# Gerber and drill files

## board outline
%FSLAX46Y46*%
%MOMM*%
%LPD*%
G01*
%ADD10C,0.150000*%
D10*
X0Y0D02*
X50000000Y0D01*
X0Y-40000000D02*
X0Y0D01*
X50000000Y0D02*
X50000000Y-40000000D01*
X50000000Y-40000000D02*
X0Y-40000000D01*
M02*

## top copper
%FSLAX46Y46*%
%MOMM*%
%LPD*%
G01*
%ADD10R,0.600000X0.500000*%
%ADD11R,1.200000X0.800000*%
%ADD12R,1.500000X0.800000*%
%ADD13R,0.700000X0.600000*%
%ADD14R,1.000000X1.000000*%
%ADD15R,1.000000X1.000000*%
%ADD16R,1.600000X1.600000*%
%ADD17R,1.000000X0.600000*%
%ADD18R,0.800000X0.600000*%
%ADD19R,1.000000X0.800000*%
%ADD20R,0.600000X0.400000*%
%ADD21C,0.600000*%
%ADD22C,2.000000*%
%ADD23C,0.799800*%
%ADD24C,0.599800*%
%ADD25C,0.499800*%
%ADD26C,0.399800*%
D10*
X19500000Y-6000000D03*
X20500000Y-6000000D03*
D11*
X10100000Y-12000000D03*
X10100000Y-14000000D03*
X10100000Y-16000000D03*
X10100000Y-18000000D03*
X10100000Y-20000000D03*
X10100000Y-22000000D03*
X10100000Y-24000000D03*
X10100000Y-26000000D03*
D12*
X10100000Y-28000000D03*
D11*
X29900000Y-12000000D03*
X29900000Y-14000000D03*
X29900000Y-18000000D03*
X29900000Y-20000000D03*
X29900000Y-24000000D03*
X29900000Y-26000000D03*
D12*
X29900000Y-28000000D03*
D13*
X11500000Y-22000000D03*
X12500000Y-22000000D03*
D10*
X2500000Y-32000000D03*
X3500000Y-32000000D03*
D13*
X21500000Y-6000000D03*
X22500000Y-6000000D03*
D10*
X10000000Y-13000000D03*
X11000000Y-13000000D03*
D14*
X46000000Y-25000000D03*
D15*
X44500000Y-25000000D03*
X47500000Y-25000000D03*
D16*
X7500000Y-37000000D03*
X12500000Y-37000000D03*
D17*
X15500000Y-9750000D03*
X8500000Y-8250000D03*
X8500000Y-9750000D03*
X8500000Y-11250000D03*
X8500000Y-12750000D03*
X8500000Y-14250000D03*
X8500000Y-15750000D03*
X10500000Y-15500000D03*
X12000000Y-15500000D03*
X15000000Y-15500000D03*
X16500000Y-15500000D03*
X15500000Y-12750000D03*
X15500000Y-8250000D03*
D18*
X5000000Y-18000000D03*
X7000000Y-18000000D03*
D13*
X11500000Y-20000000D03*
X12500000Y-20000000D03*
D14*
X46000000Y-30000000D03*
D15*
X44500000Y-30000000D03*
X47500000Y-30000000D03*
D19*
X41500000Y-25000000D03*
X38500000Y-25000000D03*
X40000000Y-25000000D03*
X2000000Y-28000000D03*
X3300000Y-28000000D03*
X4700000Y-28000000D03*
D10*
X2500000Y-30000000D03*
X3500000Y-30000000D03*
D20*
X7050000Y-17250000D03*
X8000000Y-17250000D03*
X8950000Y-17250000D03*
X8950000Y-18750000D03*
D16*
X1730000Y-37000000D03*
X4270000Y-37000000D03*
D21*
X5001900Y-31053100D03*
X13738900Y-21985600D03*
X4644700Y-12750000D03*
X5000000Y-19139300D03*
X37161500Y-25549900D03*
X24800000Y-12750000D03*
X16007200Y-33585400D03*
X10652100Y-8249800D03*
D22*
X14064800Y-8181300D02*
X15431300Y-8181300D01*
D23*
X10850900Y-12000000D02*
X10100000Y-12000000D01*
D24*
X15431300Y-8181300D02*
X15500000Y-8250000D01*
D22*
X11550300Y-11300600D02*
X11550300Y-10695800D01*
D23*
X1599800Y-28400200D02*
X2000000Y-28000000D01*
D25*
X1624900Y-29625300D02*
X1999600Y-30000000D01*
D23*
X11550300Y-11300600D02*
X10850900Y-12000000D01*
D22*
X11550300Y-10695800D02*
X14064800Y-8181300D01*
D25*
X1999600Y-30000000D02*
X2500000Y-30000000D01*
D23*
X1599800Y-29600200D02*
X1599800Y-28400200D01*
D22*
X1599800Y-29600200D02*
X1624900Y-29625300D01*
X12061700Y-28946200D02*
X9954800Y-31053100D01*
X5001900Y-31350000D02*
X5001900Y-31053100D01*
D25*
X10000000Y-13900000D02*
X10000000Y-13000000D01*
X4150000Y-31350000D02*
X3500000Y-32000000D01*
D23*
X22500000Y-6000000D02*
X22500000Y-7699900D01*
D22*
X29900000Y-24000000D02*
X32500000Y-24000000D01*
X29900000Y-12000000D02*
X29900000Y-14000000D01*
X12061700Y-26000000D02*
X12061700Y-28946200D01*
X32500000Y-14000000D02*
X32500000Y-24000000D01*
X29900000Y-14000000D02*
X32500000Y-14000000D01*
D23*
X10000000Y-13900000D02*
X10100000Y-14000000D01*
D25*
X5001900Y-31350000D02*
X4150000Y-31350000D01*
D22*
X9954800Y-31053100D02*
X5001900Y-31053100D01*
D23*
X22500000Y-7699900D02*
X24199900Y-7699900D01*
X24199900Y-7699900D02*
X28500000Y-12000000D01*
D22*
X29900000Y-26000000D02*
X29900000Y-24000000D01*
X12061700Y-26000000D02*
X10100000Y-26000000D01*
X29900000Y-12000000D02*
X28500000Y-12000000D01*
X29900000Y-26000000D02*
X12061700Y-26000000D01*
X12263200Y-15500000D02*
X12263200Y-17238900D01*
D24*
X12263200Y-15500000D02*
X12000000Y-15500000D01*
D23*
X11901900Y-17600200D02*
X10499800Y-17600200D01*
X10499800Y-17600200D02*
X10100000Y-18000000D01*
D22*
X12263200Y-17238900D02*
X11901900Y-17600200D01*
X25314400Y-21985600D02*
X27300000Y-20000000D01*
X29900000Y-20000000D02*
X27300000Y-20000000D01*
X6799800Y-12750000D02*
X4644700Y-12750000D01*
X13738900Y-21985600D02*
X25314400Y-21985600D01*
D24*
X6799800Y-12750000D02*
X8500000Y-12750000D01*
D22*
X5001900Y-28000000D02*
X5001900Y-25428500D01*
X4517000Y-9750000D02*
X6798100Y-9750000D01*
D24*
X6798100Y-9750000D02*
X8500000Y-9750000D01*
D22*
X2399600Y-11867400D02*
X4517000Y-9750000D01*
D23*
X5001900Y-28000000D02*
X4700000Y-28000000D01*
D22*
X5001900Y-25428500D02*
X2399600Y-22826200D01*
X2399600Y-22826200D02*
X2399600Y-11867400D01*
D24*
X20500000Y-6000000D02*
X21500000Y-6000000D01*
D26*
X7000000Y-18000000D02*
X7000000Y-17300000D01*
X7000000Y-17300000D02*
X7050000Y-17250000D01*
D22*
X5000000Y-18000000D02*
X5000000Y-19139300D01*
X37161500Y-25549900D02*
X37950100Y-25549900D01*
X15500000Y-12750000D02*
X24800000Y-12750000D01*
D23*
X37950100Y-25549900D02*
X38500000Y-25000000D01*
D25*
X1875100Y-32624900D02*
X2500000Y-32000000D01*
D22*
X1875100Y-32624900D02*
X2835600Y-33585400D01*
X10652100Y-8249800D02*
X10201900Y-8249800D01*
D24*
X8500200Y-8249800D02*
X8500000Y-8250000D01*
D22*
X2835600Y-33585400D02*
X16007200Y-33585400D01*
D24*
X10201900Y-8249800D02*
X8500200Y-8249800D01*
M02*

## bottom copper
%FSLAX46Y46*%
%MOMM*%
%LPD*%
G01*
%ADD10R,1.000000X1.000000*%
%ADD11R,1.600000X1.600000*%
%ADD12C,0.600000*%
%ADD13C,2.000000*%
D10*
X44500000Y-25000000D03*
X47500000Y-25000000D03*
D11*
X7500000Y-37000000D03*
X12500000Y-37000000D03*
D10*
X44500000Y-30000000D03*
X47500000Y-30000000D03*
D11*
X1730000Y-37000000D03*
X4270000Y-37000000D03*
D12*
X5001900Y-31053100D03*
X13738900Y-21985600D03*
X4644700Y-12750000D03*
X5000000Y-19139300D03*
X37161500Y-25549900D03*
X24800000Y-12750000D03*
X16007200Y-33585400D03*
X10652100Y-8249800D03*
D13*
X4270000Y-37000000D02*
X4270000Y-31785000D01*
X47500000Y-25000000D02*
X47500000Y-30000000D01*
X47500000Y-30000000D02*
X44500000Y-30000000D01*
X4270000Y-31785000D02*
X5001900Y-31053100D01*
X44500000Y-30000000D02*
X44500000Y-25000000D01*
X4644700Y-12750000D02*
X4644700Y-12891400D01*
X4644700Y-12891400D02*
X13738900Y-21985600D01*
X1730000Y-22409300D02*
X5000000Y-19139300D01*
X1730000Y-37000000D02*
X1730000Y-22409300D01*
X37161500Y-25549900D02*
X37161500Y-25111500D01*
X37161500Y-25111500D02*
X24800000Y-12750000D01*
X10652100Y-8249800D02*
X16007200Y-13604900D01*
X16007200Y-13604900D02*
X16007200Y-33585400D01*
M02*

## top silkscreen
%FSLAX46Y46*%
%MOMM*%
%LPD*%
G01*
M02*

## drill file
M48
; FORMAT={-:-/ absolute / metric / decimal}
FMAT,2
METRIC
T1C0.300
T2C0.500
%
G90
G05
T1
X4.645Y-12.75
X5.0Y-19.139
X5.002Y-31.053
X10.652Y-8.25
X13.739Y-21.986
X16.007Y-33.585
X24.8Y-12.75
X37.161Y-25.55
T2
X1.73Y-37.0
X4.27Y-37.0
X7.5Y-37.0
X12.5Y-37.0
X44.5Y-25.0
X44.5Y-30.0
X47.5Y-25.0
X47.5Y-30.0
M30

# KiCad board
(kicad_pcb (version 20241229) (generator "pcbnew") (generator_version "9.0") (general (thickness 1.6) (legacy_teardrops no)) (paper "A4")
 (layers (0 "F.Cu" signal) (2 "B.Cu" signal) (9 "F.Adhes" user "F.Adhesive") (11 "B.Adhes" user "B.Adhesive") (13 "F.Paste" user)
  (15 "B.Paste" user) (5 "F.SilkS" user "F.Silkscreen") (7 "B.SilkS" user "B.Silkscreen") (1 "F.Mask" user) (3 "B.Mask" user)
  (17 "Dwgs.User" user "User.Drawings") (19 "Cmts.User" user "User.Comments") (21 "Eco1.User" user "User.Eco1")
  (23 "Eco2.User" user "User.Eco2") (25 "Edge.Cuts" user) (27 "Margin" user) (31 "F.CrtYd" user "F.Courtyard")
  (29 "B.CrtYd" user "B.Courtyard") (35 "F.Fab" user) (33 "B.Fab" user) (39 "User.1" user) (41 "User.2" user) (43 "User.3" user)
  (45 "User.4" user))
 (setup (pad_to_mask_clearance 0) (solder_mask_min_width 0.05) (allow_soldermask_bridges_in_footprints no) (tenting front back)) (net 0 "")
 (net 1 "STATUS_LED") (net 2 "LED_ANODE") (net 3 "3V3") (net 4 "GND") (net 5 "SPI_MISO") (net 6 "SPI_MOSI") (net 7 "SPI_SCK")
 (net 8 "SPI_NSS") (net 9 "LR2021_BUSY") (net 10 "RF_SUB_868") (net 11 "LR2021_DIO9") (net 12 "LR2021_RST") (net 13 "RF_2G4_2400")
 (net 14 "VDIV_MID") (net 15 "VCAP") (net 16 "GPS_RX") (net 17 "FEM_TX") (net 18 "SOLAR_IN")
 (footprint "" (layer "F.Cu") (at 20 6)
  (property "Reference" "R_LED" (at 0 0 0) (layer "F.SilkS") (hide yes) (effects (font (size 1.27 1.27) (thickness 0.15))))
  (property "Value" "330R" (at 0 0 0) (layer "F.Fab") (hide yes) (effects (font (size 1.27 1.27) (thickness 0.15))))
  (pad "1" smd rect (at -0.5 0) (size 0.6 0.5) (layers "F.Cu" "F.Mask") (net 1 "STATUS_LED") (thermal_bridge_angle 45))
  (pad "2" smd rect (at 0.5 0) (size 0.6 0.5) (layers "F.Cu" "F.Mask") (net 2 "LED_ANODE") (thermal_bridge_angle 45)))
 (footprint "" (layer "F.Cu") (at 20 20)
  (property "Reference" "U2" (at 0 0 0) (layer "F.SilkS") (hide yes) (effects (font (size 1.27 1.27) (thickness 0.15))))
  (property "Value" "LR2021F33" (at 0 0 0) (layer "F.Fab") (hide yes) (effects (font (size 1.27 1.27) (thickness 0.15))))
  (pad "1" smd rect (at -9.9 -8) (size 1.2 0.8) (layers "F.Cu" "F.Mask") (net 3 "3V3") (thermal_bridge_angle 45))
  (pad "2" smd rect (at -9.9 -6) (size 1.2 0.8) (layers "F.Cu" "F.Mask") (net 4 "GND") (thermal_bridge_angle 45))
  (pad "3" smd rect (at -9.9 -4) (size 1.2 0.8) (layers "F.Cu" "F.Mask") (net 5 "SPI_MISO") (thermal_bridge_angle 45))
  (pad "4" smd rect (at -9.9 -2) (size 1.2 0.8) (layers "F.Cu" "F.Mask") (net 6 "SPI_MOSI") (thermal_bridge_angle 45))
  (pad "5" smd rect (at -9.9 0) (size 1.2 0.8) (layers "F.Cu" "F.Mask") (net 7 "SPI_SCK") (thermal_bridge_angle 45))
  (pad "6" smd rect (at -9.9 2) (size 1.2 0.8) (layers "F.Cu" "F.Mask") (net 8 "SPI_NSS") (thermal_bridge_angle 45))
  (pad "7" smd rect (at -9.9 4) (size 1.2 0.8) (layers "F.Cu" "F.Mask") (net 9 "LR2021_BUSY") (thermal_bridge_angle 45))
  (pad "8" smd rect (at -9.9 6) (size 1.2 0.8) (layers "F.Cu" "F.Mask") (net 4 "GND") (thermal_bridge_angle 45))
  (pad "9" smd rect (at -9.9 8) (size 1.5 0.8) (layers "F.Cu" "F.Mask") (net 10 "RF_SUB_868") (thermal_bridge_angle 45))
  (pad "10" smd rect (at 9.9 -8) (size 1.2 0.8) (layers "F.Cu" "F.Mask") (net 4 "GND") (thermal_bridge_angle 45))
  (pad "11" smd rect (at 9.9 -6) (size 1.2 0.8) (layers "F.Cu" "F.Mask") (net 4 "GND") (thermal_bridge_angle 45))
  (pad "13" smd rect (at 9.9 -2) (size 1.2 0.8) (layers "F.Cu" "F.Mask") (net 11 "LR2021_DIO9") (thermal_bridge_angle 45))
  (pad "14" smd rect (at 9.9 0) (size 1.2 0.8) (layers "F.Cu" "F.Mask") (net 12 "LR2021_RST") (thermal_bridge_angle 45))
  (pad "16" smd rect (at 9.9 4) (size 1.2 0.8) (layers "F.Cu" "F.Mask") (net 4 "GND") (thermal_bridge_angle 45))
  (pad "17" smd rect (at 9.9 6) (size 1.2 0.8) (layers "F.Cu" "F.Mask") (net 4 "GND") (thermal_bridge_angle 45))
  (pad "18" smd rect (at 9.9 8) (size 1.5 0.8) (layers "F.Cu" "F.Mask") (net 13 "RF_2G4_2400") (thermal_bridge_angle 45)))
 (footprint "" (layer "F.Cu") (at 12 22)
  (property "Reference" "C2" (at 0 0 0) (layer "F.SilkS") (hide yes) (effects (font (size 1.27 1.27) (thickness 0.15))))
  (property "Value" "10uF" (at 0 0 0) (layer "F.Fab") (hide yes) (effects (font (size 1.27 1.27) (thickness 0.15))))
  (pad "1" smd rect (at -0.5 0) (size 0.7 0.6) (layers "F.Cu" "F.Mask") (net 3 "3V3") (thermal_bridge_angle 45))
  (pad "2" smd rect (at 0.5 0) (size 0.7 0.6) (layers "F.Cu" "F.Mask") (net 4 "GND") (thermal_bridge_angle 45)))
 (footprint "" (layer "F.Cu") (at 3 32)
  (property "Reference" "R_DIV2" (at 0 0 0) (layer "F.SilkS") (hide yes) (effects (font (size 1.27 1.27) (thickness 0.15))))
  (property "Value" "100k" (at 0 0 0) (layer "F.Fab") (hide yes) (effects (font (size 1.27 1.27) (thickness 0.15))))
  (pad "1" smd rect (at -0.5 0) (size 0.6 0.5) (layers "F.Cu" "F.Mask") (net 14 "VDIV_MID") (thermal_bridge_angle 45))
  (pad "2" smd rect (at 0.5 0) (size 0.6 0.5) (layers "F.Cu" "F.Mask") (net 4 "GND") (thermal_bridge_angle 45)))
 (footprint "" (layer "F.Cu") (at 22 6)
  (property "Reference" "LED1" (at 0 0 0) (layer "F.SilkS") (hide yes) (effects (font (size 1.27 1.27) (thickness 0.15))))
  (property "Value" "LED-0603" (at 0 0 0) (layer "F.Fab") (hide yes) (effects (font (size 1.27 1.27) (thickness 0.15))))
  (pad "A" smd rect (at -0.5 0) (size 0.7 0.6) (layers "F.Cu" "F.Mask") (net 2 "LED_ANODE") (thermal_bridge_angle 45))
  (pad "K" smd rect (at 0.5 0) (size 0.7 0.6) (layers "F.Cu" "F.Mask") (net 4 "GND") (thermal_bridge_angle 45)))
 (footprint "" (layer "F.Cu") (at 10.5 13)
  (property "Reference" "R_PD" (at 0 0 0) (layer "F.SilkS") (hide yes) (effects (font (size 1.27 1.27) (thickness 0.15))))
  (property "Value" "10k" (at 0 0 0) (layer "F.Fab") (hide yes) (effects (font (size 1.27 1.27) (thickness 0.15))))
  (pad "1" smd rect (at -0.5 0) (size 0.6 0.5) (layers "F.Cu" "F.Mask") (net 4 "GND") (thermal_bridge_angle 45))
  (pad "2" smd rect (at 0.5 0) (size 0.6 0.5) (layers "F.Cu" "F.Mask") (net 5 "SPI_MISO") (thermal_bridge_angle 45)))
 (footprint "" (layer "F.Cu") (at 46 25)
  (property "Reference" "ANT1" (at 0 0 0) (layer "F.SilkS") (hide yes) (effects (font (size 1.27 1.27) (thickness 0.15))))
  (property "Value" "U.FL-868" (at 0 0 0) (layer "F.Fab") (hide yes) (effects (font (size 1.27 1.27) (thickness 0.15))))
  (pad "1" smd rect (at 0 0) (size 1 1) (layers "F.Cu" "F.Mask") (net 10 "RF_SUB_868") (thermal_bridge_angle 45))
  (pad "2" thru_hole rect (at -1.5 0) (size 1 1) (drill 0.5) (layers "*.Cu" "*.Mask") (remove_unused_layers no) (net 4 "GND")
   (thermal_bridge_angle 45))
  (pad "3" thru_hole rect (at 1.5 0) (size 1 1) (drill 0.5) (layers "*.Cu" "*.Mask") (remove_unused_layers no) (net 4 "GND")
   (thermal_bridge_angle 45)))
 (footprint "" (layer "F.Cu") (at 10 37)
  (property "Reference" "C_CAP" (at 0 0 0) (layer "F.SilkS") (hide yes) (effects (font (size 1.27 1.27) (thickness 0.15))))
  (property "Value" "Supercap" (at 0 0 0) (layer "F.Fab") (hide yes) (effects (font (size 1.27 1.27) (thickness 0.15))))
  (pad "1" thru_hole rect (at -2.5 0) (size 1.6 1.6) (drill 0.5) (layers "*.Cu" "*.Mask") (remove_unused_layers no) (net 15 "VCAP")
   (thermal_bridge_angle 45))
  (pad "2" thru_hole rect (at 2.5 0) (size 1.6 1.6) (drill 0.5) (layers "*.Cu" "*.Mask") (remove_unused_layers no) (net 4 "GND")
   (thermal_bridge_angle 45)))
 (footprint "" (layer "F.Cu") (at 12 12)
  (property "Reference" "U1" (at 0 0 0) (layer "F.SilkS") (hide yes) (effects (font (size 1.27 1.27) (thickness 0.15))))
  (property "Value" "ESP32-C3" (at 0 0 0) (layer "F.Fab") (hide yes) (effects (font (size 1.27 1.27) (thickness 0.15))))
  (pad "GND" smd rect (at 3.5 -2.25) (size 1 0.6) (layers "F.Cu" "F.Mask") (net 4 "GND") (thermal_bridge_angle 45))
  (pad "GPIO0" smd rect (at -3.5 -3.75) (size 1 0.6) (layers "F.Cu" "F.Mask") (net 14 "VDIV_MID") (thermal_bridge_angle 45))
  (pad "GPIO1" smd rect (at -3.5 -2.25) (size 1 0.6) (layers "F.Cu" "F.Mask") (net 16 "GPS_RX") (thermal_bridge_angle 45))
  (pad "GPIO2" smd rect (at -3.5 -0.75) (size 1 0.6) (layers "F.Cu" "F.Mask") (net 5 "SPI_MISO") (thermal_bridge_angle 45))
  (pad "GPIO3" smd rect (at -3.5 0.75) (size 1 0.6) (layers "F.Cu" "F.Mask") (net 12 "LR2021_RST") (thermal_bridge_angle 45))
  (pad "GPIO4" smd rect (at -3.5 2.25) (size 1 0.6) (layers "F.Cu" "F.Mask") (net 9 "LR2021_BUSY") (thermal_bridge_angle 45))
  (pad "GPIO5" smd rect (at -3.5 3.75) (size 1 0.6) (layers "F.Cu" "F.Mask") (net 11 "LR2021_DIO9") (thermal_bridge_angle 45))
  (pad "GPIO6" smd rect (at -1.5 3.5) (size 1 0.6) (layers "F.Cu" "F.Mask") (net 7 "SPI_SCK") (thermal_bridge_angle 45))
  (pad "GPIO7" smd rect (at 0 3.5) (size 1 0.6) (layers "F.Cu" "F.Mask") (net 6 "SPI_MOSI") (thermal_bridge_angle 45))
  (pad "GPIO9" smd rect (at 3 3.5) (size 1 0.6) (layers "F.Cu" "F.Mask") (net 1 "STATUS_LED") (thermal_bridge_angle 45))
  (pad "GPIO10" smd rect (at 4.5 3.5) (size 1 0.6) (layers "F.Cu" "F.Mask") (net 8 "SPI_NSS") (thermal_bridge_angle 45))
  (pad "GPIO19" smd rect (at 3.5 0.75) (size 1 0.6) (layers "F.Cu" "F.Mask") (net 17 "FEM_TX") (thermal_bridge_angle 45))
  (pad "VCC" smd rect (at 3.5 -3.75) (size 1 0.6) (layers "F.Cu" "F.Mask") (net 3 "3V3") (thermal_bridge_angle 45)))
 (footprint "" (layer "F.Cu") (at 6 18)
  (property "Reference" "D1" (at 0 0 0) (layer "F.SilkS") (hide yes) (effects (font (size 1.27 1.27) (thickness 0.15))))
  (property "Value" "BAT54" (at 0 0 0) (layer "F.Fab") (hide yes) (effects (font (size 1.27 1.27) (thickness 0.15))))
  (pad "A" smd rect (at -1 0) (size 0.8 0.6) (layers "F.Cu" "F.Mask") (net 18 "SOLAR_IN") (thermal_bridge_angle 45))
  (pad "K" smd rect (at 1 0) (size 0.8 0.6) (layers "F.Cu" "F.Mask") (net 15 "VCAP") (thermal_bridge_angle 45)))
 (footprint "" (layer "F.Cu") (at 12 20)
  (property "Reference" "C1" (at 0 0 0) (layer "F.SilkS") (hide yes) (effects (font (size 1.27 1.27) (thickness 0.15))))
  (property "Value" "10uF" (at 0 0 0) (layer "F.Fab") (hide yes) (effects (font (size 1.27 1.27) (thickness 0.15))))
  (pad "1" smd rect (at -0.5 0) (size 0.7 0.6) (layers "F.Cu" "F.Mask") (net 15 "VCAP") (thermal_bridge_angle 45))
  (pad "2" smd rect (at 0.5 0) (size 0.7 0.6) (layers "F.Cu" "F.Mask") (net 4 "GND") (thermal_bridge_angle 45)))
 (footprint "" (layer "F.Cu") (at 46 30)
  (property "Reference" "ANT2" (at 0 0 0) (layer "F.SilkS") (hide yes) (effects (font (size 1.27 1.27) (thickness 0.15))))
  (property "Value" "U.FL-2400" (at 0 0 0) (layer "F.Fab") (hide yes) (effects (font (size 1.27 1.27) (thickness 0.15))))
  (pad "1" smd rect (at 0 0) (size 1 1) (layers "F.Cu" "F.Mask") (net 13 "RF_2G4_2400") (thermal_bridge_angle 45))
  (pad "2" thru_hole rect (at -1.5 0) (size 1 1) (drill 0.5) (layers "*.Cu" "*.Mask") (remove_unused_layers no) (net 4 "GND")
   (thermal_bridge_angle 45))
  (pad "3" thru_hole rect (at 1.5 0) (size 1 1) (drill 0.5) (layers "*.Cu" "*.Mask") (remove_unused_layers no) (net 4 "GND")
   (thermal_bridge_angle 45)))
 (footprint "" (layer "F.Cu") (at 40 25)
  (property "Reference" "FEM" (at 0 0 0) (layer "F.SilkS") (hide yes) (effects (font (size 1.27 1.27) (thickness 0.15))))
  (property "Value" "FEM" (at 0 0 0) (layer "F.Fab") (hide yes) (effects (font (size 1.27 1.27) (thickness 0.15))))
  (pad "GND" smd rect (at 1.5 0) (size 1 0.8) (layers "F.Cu" "F.Mask") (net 4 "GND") (thermal_bridge_angle 45))
  (pad "TX" smd rect (at -1.5 0) (size 1 0.8) (layers "F.Cu" "F.Mask") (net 17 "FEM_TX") (thermal_bridge_angle 45))
  (pad "VCC" smd rect (at 0 0) (size 1 0.8) (layers "F.Cu" "F.Mask") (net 3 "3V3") (thermal_bridge_angle 45)))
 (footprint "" (layer "F.Cu") (at 4 28)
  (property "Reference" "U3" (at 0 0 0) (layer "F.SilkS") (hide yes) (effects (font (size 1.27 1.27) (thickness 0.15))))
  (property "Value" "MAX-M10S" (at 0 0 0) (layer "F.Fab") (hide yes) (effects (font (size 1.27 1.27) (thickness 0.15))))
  (pad "1" smd rect (at -2 0) (size 1 0.8) (layers "F.Cu" "F.Mask") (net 3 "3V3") (thermal_bridge_angle 45))
  (pad "2" smd rect (at -0.7 0) (size 1 0.8) (layers "F.Cu" "F.Mask") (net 4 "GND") (thermal_bridge_angle 45))
  (pad "3" smd rect (at 0.7 0) (size 1 0.8) (layers "F.Cu" "F.Mask") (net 16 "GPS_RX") (thermal_bridge_angle 45)))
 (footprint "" (layer "F.Cu") (at 3 30)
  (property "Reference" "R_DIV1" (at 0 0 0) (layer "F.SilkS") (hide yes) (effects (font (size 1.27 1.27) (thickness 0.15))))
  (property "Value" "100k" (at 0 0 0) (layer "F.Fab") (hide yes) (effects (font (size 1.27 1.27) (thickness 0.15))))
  (pad "1" smd rect (at -0.5 0) (size 0.6 0.5) (layers "F.Cu" "F.Mask") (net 3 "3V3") (thermal_bridge_angle 45))
  (pad "2" smd rect (at 0.5 0) (size 0.6 0.5) (layers "F.Cu" "F.Mask") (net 14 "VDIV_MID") (thermal_bridge_angle 45)))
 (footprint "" (layer "F.Cu") (at 8 18)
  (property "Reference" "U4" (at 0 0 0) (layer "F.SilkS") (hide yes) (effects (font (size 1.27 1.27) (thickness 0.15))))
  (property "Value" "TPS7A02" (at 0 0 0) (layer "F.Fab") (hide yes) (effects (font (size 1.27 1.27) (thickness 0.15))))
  (pad "1" smd rect (at -0.95 -0.75) (size 0.6 0.4) (layers "F.Cu" "F.Mask") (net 15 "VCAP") (thermal_bridge_angle 45))
  (pad "2" smd rect (at 0 -0.75) (size 0.6 0.4) (layers "F.Cu" "F.Mask") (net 4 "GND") (thermal_bridge_angle 45))
  (pad "3" smd rect (at 0.95 -0.75) (size 0.6 0.4) (layers "F.Cu" "F.Mask") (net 15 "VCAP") (thermal_bridge_angle 45))
  (pad "4" smd rect (at 0.95 0.75) (size 0.6 0.4) (layers "F.Cu" "F.Mask") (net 3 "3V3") (thermal_bridge_angle 45)))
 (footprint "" (layer "F.Cu") (at 3 37)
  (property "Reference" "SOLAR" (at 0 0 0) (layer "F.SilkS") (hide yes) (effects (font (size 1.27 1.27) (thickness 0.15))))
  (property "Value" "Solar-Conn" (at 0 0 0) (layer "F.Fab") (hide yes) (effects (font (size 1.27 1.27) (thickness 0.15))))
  (pad "1" thru_hole rect (at -1.27 0) (size 1.6 1.6) (drill 0.5) (layers "*.Cu" "*.Mask") (remove_unused_layers no) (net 18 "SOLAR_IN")
   (thermal_bridge_angle 45))
  (pad "2" thru_hole rect (at 1.27 0) (size 1.6 1.6) (drill 0.5) (layers "*.Cu" "*.Mask") (remove_unused_layers no) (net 4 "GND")
   (thermal_bridge_angle 45)))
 (gr_line (start 0 0) (end 50 0) (stroke (width 0.15) (type default)) (layer "Edge.Cuts"))
 (gr_line (start 0 40) (end 0 0) (stroke (width 0.15) (type default)) (layer "Edge.Cuts"))
 (gr_line (start 50 0) (end 50 40) (stroke (width 0.15) (type default)) (layer "Edge.Cuts"))
 (gr_line (start 50 40) (end 0 40) (stroke (width 0.15) (type default)) (layer "Edge.Cuts"))
 (segment (start 14.0648 8.1813) (end 15.4313 8.1813) (width 2) (layer "F.Cu") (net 3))
 (segment (start 10.8509 12) (end 10.1 12) (width 0.7998) (layer "F.Cu") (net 3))
 (segment (start 15.4313 8.1813) (end 15.5 8.25) (width 0.5998) (layer "F.Cu") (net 3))
 (segment (start 11.5503 11.3006) (end 11.5503 10.6958) (width 2) (layer "F.Cu") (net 3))
 (segment (start 1.5998 28.4002) (end 2 28) (width 0.7998) (layer "F.Cu") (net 3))
 (segment (start 1.6249 29.6253) (end 1.9996 30) (width 0.4998) (layer "F.Cu") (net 3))
 (segment (start 11.5503 11.3006) (end 10.8509 12) (width 0.7998) (layer "F.Cu") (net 3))
 (segment (start 11.5503 10.6958) (end 14.0648 8.1813) (width 2) (layer "F.Cu") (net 3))
 (segment (start 1.9996 30) (end 2.5 30) (width 0.4998) (layer "F.Cu") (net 3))
 (segment (start 1.5998 29.6002) (end 1.5998 28.4002) (width 0.7998) (layer "F.Cu") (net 3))
 (segment (start 1.5998 29.6002) (end 1.6249 29.6253) (width 2) (layer "F.Cu") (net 3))
 (segment (start 12.0617 28.9462) (end 9.9548 31.0531) (width 2) (layer "F.Cu") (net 4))
 (segment (start 5.0019 31.35) (end 5.0019 31.0531) (width 2) (layer "F.Cu") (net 4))
 (segment (start 10 13.9) (end 10 13) (width 0.4998) (layer "F.Cu") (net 4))
 (segment (start 4.15 31.35) (end 3.5 32) (width 0.4998) (layer "F.Cu") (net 4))
 (segment (start 22.5 6) (end 22.5 7.6999) (width 0.7998) (layer "F.Cu") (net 4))
 (segment (start 29.9 24) (end 32.5 24) (width 2) (layer "F.Cu") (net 4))
 (segment (start 29.9 12) (end 29.9 14) (width 2) (layer "F.Cu") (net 4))
 (segment (start 12.0617 26) (end 12.0617 28.9462) (width 2) (layer "F.Cu") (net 4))
 (segment (start 32.5 14) (end 32.5 24) (width 2) (layer "F.Cu") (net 4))
 (segment (start 29.9 14) (end 32.5 14) (width 2) (layer "F.Cu") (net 4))
 (segment (start 10 13.9) (end 10.1 14) (width 0.7998) (layer "F.Cu") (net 4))
 (segment (start 5.0019 31.35) (end 4.15 31.35) (width 0.4998) (layer "F.Cu") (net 4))
 (segment (start 9.9548 31.0531) (end 5.0019 31.0531) (width 2) (layer "F.Cu") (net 4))
 (segment (start 22.5 7.6999) (end 24.1999 7.6999) (width 0.7998) (layer "F.Cu") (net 4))
 (segment (start 24.1999 7.6999) (end 28.5 12) (width 0.7998) (layer "F.Cu") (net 4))
 (segment (start 29.9 26) (end 29.9 24) (width 2) (layer "F.Cu") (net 4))
 (segment (start 12.0617 26) (end 10.1 26) (width 2) (layer "F.Cu") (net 4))
 (segment (start 29.9 12) (end 28.5 12) (width 2) (layer "F.Cu") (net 4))
 (segment (start 29.9 26) (end 12.0617 26) (width 2) (layer "F.Cu") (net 4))
 (via (at 5.0019 31.0531) (size 0.6) (drill 0.3) (layers "F.Cu" "B.Cu") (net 4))
 (segment (start 4.27 37) (end 4.27 31.785) (width 2) (layer "B.Cu") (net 4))
 (segment (start 47.5 25) (end 47.5 30) (width 2) (layer "B.Cu") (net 4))
 (segment (start 47.5 30) (end 44.5 30) (width 2) (layer "B.Cu") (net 4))
 (segment (start 4.27 31.785) (end 5.0019 31.0531) (width 2) (layer "B.Cu") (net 4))
 (segment (start 44.5 30) (end 44.5 25) (width 2) (layer "B.Cu") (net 4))
 (segment (start 12.2632 15.5) (end 12.2632 17.2389) (width 2) (layer "F.Cu") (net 6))
 (segment (start 12.2632 15.5) (end 12 15.5) (width 0.5998) (layer "F.Cu") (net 6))
 (segment (start 11.9019 17.6002) (end 10.4998 17.6002) (width 0.7998) (layer "F.Cu") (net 6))
 (segment (start 10.4998 17.6002) (end 10.1 18) (width 0.7998) (layer "F.Cu") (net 6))
 (segment (start 12.2632 17.2389) (end 11.9019 17.6002) (width 2) (layer "F.Cu") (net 6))
 (segment (start 25.3144 21.9856) (end 27.3 20) (width 2) (layer "F.Cu") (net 12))
 (segment (start 29.9 20) (end 27.3 20) (width 2) (layer "F.Cu") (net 12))
 (segment (start 6.7998 12.75) (end 4.6447 12.75) (width 2) (layer "F.Cu") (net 12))
 (segment (start 13.7389 21.9856) (end 25.3144 21.9856) (width 2) (layer "F.Cu") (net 12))
 (segment (start 6.7998 12.75) (end 8.5 12.75) (width 0.5998) (layer "F.Cu") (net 12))
 (via (at 13.7389 21.9856) (size 0.6) (drill 0.3) (layers "F.Cu" "B.Cu") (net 12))
 (via (at 4.6447 12.75) (size 0.6) (drill 0.3) (layers "F.Cu" "B.Cu") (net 12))
 (segment (start 4.6447 12.75) (end 4.6447 12.8914) (width 2) (layer "B.Cu") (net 12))
 (segment (start 4.6447 12.8914) (end 13.7389 21.9856) (width 2) (layer "B.Cu") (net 12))
 (segment (start 5.0019 28) (end 5.0019 25.4285) (width 2) (layer "F.Cu") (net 16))
 (segment (start 4.517 9.75) (end 6.7981 9.75) (width 2) (layer "F.Cu") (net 16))
 (segment (start 6.7981 9.75) (end 8.5 9.75) (width 0.5998) (layer "F.Cu") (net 16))
 (segment (start 2.3996 11.8674) (end 4.517 9.75) (width 2) (layer "F.Cu") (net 16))
 (segment (start 5.0019 28) (end 4.7 28) (width 0.7998) (layer "F.Cu") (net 16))
 (segment (start 5.0019 25.4285) (end 2.3996 22.8262) (width 2) (layer "F.Cu") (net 16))
 (segment (start 2.3996 22.8262) (end 2.3996 11.8674) (width 2) (layer "F.Cu") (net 16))
 (segment (start 20.5 6) (end 21.5 6) (width 0.5998) (layer "F.Cu") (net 2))
 (segment (start 7 18) (end 7 17.3) (width 0.3998) (layer "F.Cu") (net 15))
 (segment (start 7 17.3) (end 7.05 17.25) (width 0.3998) (layer "F.Cu") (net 15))
 (segment (start 5 18) (end 5 19.1393) (width 2) (layer "F.Cu") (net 18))
 (via (at 5 19.1393) (size 0.6) (drill 0.3) (layers "F.Cu" "B.Cu") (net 18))
 (segment (start 1.73 22.4093) (end 5 19.1393) (width 2) (layer "B.Cu") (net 18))
 (segment (start 1.73 37) (end 1.73 22.4093) (width 2) (layer "B.Cu") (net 18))
 (segment (start 37.1615 25.5499) (end 37.9501 25.5499) (width 2) (layer "F.Cu") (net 17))
 (segment (start 15.5 12.75) (end 24.8 12.75) (width 2) (layer "F.Cu") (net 17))
 (segment (start 37.9501 25.5499) (end 38.5 25) (width 0.7998) (layer "F.Cu") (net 17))
 (via (at 37.1615 25.5499) (size 0.6) (drill 0.3) (layers "F.Cu" "B.Cu") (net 17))
 (via (at 24.8 12.75) (size 0.6) (drill 0.3) (layers "F.Cu" "B.Cu") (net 17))
 (segment (start 37.1615 25.5499) (end 37.1615 25.1115) (width 2) (layer "B.Cu") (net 17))
 (segment (start 37.1615 25.1115) (end 24.8 12.75) (width 2) (layer "B.Cu") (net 17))
 (segment (start 1.8751 32.6249) (end 2.5 32) (width 0.4998) (layer "F.Cu") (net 14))
 (segment (start 1.8751 32.6249) (end 2.8356 33.5854) (width 2) (layer "F.Cu") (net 14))
 (segment (start 10.6521 8.2498) (end 10.2019 8.2498) (width 2) (layer "F.Cu") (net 14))
 (segment (start 8.5002 8.2498) (end 8.5 8.25) (width 0.5998) (layer "F.Cu") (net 14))
 (segment (start 2.8356 33.5854) (end 16.0072 33.5854) (width 2) (layer "F.Cu") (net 14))
 (segment (start 10.2019 8.2498) (end 8.5002 8.2498) (width 0.5998) (layer "F.Cu") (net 14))
 (via (at 16.0072 33.5854) (size 0.6) (drill 0.3) (layers "F.Cu" "B.Cu") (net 14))
 (via (at 10.6521 8.2498) (size 0.6) (drill 0.3) (layers "F.Cu" "B.Cu") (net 14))
 (segment (start 10.6521 8.2498) (end 16.0072 13.6049) (width 2) (layer "B.Cu") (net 14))
 (segment (start 16.0072 13.6049) (end 16.0072 33.5854) (width 2) (layer "B.Cu") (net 14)))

